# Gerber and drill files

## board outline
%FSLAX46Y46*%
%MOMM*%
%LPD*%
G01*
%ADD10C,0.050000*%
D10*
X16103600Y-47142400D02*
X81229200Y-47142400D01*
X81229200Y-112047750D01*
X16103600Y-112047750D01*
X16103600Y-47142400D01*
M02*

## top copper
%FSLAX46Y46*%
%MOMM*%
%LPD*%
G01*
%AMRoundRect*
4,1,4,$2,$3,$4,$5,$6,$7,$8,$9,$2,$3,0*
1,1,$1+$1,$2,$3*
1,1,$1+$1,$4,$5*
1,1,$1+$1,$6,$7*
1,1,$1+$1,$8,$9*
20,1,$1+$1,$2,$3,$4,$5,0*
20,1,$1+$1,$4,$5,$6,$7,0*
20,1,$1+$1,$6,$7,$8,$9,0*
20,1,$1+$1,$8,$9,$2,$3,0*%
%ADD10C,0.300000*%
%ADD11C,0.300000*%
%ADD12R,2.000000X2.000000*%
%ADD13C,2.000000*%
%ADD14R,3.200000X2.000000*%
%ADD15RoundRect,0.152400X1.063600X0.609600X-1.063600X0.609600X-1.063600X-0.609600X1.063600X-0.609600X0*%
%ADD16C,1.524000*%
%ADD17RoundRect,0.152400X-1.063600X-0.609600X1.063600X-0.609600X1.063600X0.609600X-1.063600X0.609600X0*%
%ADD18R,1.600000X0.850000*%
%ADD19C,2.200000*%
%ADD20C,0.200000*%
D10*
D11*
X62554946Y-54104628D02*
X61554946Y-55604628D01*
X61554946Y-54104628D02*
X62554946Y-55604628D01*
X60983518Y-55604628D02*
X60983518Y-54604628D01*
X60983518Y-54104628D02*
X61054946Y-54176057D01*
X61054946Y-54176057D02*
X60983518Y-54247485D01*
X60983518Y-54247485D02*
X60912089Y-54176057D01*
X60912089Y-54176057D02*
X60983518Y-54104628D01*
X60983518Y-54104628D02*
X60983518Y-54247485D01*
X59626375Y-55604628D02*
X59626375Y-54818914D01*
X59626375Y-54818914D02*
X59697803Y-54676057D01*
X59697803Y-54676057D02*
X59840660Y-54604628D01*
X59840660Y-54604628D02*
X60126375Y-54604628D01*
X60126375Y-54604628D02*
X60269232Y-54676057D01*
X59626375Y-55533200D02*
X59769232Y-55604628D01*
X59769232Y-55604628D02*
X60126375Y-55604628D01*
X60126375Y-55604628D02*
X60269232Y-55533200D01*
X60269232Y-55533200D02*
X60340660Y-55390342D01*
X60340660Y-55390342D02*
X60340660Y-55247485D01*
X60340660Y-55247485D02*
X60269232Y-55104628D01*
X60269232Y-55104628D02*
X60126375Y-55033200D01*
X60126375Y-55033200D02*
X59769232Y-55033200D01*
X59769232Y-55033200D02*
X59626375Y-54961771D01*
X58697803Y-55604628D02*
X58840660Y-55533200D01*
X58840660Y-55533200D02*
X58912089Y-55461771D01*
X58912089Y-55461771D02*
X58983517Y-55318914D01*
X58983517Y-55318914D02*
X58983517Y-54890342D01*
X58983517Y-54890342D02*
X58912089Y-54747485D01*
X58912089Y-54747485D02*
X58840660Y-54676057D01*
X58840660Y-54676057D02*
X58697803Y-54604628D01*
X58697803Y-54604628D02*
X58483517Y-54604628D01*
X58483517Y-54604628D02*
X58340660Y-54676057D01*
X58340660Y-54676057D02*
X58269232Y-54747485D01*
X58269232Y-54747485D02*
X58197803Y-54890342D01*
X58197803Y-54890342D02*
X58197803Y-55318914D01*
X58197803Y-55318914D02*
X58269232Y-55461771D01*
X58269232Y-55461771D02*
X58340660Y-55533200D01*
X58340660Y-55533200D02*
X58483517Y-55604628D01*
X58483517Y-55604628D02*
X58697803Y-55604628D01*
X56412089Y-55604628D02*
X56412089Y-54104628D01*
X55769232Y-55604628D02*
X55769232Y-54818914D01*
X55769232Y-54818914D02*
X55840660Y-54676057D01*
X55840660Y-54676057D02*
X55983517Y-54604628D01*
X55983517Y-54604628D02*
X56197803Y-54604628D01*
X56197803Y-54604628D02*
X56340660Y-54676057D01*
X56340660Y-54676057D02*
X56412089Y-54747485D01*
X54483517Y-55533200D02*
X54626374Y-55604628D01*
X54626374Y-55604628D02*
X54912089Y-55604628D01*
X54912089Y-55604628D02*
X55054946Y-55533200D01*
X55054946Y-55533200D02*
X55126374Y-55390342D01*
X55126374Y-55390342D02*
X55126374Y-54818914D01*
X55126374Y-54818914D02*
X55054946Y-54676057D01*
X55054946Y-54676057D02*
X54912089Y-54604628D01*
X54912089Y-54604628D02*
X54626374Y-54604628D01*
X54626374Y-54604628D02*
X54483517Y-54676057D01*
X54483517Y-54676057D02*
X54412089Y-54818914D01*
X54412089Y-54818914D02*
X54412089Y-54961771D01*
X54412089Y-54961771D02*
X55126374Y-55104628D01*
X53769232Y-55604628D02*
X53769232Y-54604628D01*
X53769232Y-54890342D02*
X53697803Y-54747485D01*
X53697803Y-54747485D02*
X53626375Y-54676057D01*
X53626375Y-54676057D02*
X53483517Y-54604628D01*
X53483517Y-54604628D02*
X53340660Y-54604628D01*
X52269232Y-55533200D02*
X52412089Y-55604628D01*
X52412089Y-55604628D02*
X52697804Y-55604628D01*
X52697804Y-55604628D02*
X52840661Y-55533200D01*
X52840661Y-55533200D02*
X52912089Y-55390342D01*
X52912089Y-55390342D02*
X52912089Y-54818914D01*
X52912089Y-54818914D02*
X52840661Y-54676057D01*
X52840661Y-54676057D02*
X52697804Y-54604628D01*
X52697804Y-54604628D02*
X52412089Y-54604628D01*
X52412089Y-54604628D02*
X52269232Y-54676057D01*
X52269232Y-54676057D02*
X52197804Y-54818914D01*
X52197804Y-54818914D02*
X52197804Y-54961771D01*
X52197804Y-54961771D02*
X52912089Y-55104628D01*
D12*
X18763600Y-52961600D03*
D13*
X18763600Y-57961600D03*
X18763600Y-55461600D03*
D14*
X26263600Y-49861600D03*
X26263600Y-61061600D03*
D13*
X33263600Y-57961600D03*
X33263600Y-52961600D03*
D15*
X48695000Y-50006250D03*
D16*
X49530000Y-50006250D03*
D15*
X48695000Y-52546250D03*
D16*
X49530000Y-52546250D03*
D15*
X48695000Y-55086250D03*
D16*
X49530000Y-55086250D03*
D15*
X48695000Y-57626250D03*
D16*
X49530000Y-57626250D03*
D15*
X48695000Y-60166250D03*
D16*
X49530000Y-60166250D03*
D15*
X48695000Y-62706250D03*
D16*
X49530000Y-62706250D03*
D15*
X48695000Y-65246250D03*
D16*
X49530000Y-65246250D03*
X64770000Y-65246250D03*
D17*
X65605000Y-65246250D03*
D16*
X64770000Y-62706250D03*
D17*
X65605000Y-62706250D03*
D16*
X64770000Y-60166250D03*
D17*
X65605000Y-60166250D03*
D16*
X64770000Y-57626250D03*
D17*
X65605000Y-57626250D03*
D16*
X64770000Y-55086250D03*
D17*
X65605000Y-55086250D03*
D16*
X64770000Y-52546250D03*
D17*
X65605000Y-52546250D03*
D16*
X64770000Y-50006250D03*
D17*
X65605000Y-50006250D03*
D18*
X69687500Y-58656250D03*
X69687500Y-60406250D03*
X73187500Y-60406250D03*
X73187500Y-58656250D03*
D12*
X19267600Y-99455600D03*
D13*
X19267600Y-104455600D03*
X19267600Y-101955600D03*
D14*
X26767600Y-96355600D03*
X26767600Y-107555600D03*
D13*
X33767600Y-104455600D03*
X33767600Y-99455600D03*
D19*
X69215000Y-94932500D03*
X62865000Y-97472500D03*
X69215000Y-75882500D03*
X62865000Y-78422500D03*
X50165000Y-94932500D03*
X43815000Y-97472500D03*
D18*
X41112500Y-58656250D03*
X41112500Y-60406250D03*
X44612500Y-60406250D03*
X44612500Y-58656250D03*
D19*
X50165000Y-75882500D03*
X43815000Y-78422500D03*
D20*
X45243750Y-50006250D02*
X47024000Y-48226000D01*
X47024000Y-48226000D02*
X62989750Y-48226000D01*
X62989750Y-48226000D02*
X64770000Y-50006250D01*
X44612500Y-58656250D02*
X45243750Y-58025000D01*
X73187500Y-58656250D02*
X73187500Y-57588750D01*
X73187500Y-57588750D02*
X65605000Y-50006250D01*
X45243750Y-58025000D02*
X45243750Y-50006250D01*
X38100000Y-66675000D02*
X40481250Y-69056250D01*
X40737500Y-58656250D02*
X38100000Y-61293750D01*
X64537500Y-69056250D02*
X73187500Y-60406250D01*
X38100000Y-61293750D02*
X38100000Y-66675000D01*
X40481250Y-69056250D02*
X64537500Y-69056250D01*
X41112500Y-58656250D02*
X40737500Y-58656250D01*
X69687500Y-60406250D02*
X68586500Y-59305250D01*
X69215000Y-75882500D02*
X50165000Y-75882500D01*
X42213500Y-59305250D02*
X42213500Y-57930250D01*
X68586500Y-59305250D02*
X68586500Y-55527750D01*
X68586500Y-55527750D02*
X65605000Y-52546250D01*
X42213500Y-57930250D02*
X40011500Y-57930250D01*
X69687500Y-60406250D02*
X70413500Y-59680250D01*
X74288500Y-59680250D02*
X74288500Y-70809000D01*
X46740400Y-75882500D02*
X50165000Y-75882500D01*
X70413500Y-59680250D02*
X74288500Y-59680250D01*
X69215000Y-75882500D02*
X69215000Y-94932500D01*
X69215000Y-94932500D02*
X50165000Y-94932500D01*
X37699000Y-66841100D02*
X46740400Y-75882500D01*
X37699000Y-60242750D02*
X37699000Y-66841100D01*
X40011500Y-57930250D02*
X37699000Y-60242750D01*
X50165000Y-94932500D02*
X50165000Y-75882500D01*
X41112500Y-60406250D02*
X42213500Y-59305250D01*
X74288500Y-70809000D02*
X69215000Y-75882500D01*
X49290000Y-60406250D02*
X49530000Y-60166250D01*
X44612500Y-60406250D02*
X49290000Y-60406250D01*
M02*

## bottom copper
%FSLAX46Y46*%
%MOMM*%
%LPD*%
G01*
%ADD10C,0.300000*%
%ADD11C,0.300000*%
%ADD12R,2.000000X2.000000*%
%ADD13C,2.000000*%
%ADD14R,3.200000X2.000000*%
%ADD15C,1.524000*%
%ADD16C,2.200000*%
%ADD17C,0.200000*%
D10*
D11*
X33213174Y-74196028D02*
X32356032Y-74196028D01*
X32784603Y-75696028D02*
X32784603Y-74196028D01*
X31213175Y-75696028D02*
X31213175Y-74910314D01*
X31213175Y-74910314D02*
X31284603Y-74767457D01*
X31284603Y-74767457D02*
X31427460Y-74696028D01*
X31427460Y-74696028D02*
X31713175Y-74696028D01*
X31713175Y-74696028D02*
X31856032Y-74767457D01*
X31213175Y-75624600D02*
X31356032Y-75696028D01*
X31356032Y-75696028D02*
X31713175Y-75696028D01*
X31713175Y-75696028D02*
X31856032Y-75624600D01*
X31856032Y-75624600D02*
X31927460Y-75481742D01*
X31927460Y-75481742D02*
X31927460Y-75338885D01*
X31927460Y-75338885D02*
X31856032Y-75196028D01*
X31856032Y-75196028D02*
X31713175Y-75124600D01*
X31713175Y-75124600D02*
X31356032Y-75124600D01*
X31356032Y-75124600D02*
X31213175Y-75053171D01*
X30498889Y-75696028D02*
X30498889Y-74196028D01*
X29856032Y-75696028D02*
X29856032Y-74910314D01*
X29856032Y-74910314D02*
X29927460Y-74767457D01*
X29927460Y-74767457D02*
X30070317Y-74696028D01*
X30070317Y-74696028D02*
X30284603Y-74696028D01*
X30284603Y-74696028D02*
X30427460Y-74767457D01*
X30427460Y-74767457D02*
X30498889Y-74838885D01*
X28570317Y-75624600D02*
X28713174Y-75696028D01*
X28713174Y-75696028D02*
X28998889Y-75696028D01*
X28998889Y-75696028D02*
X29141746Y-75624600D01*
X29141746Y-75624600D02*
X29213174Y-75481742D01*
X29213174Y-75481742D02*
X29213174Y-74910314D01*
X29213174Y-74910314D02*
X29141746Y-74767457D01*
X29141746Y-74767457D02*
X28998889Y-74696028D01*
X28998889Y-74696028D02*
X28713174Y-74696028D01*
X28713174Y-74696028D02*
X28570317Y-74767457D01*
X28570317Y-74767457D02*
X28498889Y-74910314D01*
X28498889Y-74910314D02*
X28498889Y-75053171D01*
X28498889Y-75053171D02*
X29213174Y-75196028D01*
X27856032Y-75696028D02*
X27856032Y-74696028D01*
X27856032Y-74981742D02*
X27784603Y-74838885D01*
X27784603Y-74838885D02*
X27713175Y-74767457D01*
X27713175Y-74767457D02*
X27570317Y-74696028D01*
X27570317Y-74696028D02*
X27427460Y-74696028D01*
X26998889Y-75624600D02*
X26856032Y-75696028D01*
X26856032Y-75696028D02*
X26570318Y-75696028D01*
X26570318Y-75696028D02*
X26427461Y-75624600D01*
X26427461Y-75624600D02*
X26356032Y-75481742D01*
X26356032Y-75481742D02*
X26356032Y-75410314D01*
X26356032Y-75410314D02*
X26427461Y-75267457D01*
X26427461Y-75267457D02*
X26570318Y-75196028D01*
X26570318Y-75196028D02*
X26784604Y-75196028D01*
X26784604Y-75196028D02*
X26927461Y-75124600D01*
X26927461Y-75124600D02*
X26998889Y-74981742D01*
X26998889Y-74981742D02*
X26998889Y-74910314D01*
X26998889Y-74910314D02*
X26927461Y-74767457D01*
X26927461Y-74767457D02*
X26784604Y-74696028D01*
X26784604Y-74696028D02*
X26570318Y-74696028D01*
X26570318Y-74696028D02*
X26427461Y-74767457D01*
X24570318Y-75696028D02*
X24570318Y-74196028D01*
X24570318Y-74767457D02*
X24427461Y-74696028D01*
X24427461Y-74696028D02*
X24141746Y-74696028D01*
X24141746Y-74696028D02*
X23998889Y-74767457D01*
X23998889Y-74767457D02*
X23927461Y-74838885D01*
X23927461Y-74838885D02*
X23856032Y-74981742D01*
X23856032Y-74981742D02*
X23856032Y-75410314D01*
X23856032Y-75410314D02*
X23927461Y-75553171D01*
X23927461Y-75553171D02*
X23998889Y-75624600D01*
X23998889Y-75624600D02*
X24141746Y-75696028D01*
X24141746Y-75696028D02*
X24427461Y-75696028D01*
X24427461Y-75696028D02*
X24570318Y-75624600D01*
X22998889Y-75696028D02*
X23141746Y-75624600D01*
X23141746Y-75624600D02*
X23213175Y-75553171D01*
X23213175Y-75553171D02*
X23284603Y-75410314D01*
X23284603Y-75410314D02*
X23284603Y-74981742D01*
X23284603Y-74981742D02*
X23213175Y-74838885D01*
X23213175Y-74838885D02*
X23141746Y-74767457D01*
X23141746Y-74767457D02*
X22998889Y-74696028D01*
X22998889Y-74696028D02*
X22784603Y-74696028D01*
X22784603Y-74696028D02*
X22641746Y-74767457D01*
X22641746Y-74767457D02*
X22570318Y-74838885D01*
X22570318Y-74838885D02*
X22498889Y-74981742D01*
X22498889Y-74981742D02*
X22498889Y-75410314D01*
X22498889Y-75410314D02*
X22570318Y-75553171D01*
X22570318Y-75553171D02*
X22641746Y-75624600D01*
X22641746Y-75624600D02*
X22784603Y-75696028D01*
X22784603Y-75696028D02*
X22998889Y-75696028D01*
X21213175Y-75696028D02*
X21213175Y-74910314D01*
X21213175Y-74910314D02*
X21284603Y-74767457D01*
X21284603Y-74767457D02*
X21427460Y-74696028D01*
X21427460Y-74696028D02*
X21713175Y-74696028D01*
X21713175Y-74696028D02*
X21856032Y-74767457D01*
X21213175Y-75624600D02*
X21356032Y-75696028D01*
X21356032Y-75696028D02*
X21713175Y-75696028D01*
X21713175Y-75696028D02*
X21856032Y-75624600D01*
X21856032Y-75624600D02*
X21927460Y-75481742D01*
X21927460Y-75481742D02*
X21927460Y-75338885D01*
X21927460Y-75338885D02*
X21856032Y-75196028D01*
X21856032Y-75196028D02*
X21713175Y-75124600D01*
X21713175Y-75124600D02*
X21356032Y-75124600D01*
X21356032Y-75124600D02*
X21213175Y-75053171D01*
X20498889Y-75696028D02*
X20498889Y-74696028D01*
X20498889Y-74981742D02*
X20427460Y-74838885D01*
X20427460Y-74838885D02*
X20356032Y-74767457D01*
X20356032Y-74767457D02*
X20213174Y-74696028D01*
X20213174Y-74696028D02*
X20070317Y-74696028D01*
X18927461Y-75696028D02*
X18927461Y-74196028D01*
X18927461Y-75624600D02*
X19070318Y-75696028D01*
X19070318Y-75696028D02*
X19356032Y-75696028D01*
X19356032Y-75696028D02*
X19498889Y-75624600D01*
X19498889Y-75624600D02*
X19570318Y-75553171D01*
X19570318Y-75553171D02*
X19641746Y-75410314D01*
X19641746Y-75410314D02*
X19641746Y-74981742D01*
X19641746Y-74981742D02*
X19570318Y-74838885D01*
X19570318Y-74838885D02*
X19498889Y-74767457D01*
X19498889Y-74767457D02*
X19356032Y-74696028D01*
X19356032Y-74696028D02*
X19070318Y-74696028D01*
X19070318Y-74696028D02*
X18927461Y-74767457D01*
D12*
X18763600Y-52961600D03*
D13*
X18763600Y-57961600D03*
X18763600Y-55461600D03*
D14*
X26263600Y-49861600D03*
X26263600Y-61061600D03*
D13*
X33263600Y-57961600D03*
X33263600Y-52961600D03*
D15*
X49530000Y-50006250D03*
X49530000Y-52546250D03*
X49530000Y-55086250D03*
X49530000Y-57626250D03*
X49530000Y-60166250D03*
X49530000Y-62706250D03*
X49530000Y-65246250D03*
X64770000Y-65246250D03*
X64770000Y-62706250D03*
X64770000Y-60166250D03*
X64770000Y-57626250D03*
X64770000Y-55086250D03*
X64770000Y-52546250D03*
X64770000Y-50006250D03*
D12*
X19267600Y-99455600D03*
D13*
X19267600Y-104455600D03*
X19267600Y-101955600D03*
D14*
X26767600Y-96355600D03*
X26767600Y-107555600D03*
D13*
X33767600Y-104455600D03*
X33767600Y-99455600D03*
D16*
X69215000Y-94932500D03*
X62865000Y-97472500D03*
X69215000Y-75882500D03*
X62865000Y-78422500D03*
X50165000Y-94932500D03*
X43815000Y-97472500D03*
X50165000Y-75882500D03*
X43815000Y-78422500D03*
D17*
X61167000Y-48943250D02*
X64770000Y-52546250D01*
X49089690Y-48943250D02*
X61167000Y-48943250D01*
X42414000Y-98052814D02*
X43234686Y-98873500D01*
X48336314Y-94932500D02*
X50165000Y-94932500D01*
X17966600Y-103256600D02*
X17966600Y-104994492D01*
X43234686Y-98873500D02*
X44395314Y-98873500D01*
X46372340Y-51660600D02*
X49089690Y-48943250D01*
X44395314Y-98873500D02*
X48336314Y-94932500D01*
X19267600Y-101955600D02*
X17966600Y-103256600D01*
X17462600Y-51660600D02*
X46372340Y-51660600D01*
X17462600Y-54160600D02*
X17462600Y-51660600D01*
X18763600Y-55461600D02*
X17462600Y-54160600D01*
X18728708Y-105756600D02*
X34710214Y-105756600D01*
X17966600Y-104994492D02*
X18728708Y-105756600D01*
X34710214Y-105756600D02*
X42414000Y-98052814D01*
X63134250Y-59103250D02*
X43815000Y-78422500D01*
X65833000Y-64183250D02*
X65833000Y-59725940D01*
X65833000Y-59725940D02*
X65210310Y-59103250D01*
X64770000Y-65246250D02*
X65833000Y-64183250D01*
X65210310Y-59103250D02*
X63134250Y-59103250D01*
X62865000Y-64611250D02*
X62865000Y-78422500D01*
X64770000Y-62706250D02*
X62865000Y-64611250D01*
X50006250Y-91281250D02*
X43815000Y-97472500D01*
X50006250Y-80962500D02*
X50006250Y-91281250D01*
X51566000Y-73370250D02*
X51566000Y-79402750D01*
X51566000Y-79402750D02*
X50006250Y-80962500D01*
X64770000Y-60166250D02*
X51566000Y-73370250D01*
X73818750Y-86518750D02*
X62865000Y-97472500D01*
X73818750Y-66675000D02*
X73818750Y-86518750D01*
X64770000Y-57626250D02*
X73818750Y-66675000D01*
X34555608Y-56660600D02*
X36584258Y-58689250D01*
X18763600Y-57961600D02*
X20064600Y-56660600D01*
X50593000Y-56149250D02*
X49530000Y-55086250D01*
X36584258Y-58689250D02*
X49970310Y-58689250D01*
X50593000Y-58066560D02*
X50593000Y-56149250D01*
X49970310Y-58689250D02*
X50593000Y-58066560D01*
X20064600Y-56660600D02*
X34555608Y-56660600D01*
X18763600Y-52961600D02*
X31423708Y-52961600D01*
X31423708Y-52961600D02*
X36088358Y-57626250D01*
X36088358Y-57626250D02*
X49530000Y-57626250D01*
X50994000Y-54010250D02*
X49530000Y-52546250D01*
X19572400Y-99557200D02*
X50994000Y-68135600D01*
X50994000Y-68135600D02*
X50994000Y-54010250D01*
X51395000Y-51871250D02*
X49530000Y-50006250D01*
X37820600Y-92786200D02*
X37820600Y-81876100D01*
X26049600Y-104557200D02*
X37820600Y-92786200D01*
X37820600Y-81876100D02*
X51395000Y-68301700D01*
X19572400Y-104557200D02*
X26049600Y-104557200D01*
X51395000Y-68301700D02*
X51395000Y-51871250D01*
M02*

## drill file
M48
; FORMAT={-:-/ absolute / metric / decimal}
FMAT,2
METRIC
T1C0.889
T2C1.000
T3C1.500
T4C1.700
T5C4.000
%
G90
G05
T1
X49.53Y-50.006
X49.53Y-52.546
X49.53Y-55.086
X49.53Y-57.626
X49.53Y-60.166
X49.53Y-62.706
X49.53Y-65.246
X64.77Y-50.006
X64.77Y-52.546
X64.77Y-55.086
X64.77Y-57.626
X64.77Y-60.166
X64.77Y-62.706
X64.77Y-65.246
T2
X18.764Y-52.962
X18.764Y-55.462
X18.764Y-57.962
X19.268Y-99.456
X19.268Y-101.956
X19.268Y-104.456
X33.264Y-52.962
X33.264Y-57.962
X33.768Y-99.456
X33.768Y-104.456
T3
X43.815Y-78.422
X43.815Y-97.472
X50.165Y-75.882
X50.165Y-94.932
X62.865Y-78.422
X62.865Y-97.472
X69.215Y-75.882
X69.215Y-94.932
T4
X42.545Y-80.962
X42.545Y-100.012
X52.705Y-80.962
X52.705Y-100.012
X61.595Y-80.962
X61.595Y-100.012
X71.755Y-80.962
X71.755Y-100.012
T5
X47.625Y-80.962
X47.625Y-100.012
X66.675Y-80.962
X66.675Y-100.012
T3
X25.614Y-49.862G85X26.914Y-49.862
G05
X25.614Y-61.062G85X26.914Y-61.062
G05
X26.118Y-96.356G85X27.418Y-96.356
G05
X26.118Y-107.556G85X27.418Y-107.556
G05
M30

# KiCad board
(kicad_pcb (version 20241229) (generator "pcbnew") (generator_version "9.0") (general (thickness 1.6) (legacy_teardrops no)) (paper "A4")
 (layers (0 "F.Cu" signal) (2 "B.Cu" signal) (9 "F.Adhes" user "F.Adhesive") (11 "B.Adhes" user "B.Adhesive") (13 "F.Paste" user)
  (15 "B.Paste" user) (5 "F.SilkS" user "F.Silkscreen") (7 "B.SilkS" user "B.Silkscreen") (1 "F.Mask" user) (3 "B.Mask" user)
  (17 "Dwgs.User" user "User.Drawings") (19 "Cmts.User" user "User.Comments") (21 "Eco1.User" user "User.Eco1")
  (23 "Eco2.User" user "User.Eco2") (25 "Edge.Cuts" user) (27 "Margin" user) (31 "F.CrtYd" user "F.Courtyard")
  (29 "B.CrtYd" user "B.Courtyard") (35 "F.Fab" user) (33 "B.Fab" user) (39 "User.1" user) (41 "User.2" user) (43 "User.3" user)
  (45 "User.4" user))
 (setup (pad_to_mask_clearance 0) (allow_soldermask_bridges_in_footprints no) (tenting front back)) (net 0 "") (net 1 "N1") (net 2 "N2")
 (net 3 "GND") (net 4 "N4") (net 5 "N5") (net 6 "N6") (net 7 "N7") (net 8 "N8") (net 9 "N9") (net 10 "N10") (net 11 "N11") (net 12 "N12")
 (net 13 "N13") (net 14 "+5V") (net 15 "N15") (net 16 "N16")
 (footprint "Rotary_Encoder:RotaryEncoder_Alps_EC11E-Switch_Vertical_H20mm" (layer "F.Cu") (at 18.7636 52.9616)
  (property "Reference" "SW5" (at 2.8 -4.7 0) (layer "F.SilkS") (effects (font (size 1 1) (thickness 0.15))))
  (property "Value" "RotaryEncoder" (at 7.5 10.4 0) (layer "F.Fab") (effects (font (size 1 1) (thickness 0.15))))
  (pad "A" thru_hole rect (at 0 0) (size 2 2) (drill 1) (layers "*.Cu" "*.Mask") (remove_unused_layers no) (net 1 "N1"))
  (pad "B" thru_hole circle (at 0 5) (size 2 2) (drill 1) (layers "*.Cu" "*.Mask") (remove_unused_layers no) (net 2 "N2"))
  (pad "C" thru_hole circle (at 0 2.5) (size 2 2) (drill 1) (layers "*.Cu" "*.Mask") (remove_unused_layers no) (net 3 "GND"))
  (pad "MP" thru_hole rect (at 7.5 -3.1) (size 3.2 2) (drill oval 2.8 1.5) (layers "*.Cu" "*.Mask") (remove_unused_layers no))
  (pad "MP" thru_hole rect (at 7.5 8.1) (size 3.2 2) (drill oval 2.8 1.5) (layers "*.Cu" "*.Mask") (remove_unused_layers no))
  (pad "S1" thru_hole circle (at 14.5 5) (size 2 2) (drill 1) (layers "*.Cu" "*.Mask") (remove_unused_layers no))
  (pad "S2" thru_hole circle (at 14.5 0) (size 2 2) (drill 1) (layers "*.Cu" "*.Mask") (remove_unused_layers no)))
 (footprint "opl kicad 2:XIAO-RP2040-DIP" (layer "F.Cu") (at 57.15 57.62625)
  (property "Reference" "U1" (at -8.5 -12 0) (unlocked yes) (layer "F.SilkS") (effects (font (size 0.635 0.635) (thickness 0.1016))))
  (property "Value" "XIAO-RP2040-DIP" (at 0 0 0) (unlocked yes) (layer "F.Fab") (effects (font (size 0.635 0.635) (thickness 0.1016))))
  (pad "1" smd roundrect (at -8.455 -7.62 180) (size 2.432 1.524) (layers "F.Cu" "F.Mask") (roundrect_rratio 0.1) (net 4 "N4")
   (thermal_bridge_angle 45))
  (pad "1" thru_hole circle (at -7.62 -7.62 180) (size 1.524 1.524) (drill 0.889) (layers "*.Cu" "*.Mask") (remove_unused_layers no)
   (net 4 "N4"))
  (pad "2" smd roundrect (at -8.455 -5.08 180) (size 2.432 1.524) (layers "F.Cu" "F.Mask") (roundrect_rratio 0.1) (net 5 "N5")
   (thermal_bridge_angle 45))
  (pad "2" thru_hole circle (at -7.62 -5.08 180) (size 1.524 1.524) (drill 0.889) (layers "*.Cu" "*.Mask") (remove_unused_layers no)
   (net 5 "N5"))
  (pad "3" smd roundrect (at -8.455 -2.54 180) (size 2.432 1.524) (layers "F.Cu" "F.Mask") (roundrect_rratio 0.1) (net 2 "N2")
   (thermal_bridge_angle 45))
  (pad "3" thru_hole circle (at -7.62 -2.54 180) (size 1.524 1.524) (drill 0.889) (layers "*.Cu" "*.Mask") (remove_unused_layers no)
   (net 2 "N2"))
  (pad "4" smd roundrect (at -8.455 0 180) (size 2.432 1.524) (layers "F.Cu" "F.Mask") (roundrect_rratio 0.1) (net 1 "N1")
   (thermal_bridge_angle 45))
  (pad "4" thru_hole circle (at -7.62 0 180) (size 1.524 1.524) (drill 0.889) (layers "*.Cu" "*.Mask") (remove_unused_layers no)
   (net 1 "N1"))
  (pad "5" smd roundrect (at -8.455 2.54 180) (size 2.432 1.524) (layers "F.Cu" "F.Mask") (roundrect_rratio 0.1) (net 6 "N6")
   (thermal_bridge_angle 45))
  (pad "5" thru_hole circle (at -7.62 2.54 180) (size 1.524 1.524) (drill 0.889) (layers "*.Cu" "*.Mask") (remove_unused_layers no)
   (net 6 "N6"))
  (pad "6" smd roundrect (at -8.455 5.08 180) (size 2.432 1.524) (layers "F.Cu" "F.Mask") (roundrect_rratio 0.1) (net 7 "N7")
   (thermal_bridge_angle 45))
  (pad "6" thru_hole circle (at -7.62 5.08 180) (size 1.524 1.524) (drill 0.889) (layers "*.Cu" "*.Mask") (remove_unused_layers no)
   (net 7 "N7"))
  (pad "7" smd roundrect (at -8.455 7.62 180) (size 2.432 1.524) (layers "F.Cu" "F.Mask") (roundrect_rratio 0.1) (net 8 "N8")
   (thermal_bridge_angle 45))
  (pad "7" thru_hole circle (at -7.62 7.62 180) (size 1.524 1.524) (drill 0.889) (layers "*.Cu" "*.Mask") (remove_unused_layers no)
   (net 8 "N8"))
  (pad "8" thru_hole circle (at 7.62 7.62) (size 1.524 1.524) (drill 0.889) (layers "*.Cu" "*.Mask") (remove_unused_layers no) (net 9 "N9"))
  (pad "8" smd roundrect (at 8.455 7.62) (size 2.432 1.524) (layers "F.Cu" "F.Mask") (roundrect_rratio 0.1) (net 9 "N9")
   (thermal_bridge_angle 45))
  (pad "9" thru_hole circle (at 7.62 5.08) (size 1.524 1.524) (drill 0.889) (layers "*.Cu" "*.Mask") (remove_unused_layers no)
   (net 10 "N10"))
  (pad "9" smd roundrect (at 8.455 5.08) (size 2.432 1.524) (layers "F.Cu" "F.Mask") (roundrect_rratio 0.1) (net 10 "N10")
   (thermal_bridge_angle 45))
  (pad "10" thru_hole circle (at 7.62 2.54) (size 1.524 1.524) (drill 0.889) (layers "*.Cu" "*.Mask") (remove_unused_layers no)
   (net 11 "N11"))
  (pad "10" smd roundrect (at 8.455 2.54) (size 2.432 1.524) (layers "F.Cu" "F.Mask") (roundrect_rratio 0.1) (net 11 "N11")
   (thermal_bridge_angle 45))
  (pad "11" thru_hole circle (at 7.62 0) (size 1.524 1.524) (drill 0.889) (layers "*.Cu" "*.Mask") (remove_unused_layers no) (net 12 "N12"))
  (pad "11" smd roundrect (at 8.455 0) (size 2.432 1.524) (layers "F.Cu" "F.Mask") (roundrect_rratio 0.1) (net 12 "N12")
   (thermal_bridge_angle 45))
  (pad "12" thru_hole circle (at 7.62 -2.54) (size 1.524 1.524) (drill 0.889) (layers "*.Cu" "*.Mask") (remove_unused_layers no)
   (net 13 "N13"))
  (pad "12" smd roundrect (at 8.455 -2.54) (size 2.432 1.524) (layers "F.Cu" "F.Mask") (roundrect_rratio 0.1) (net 13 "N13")
   (thermal_bridge_angle 45))
  (pad "13" thru_hole circle (at 7.62 -5.08) (size 1.524 1.524) (drill 0.889) (layers "*.Cu" "*.Mask") (remove_unused_layers no)
   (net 3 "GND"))
  (pad "13" smd roundrect (at 8.455 -5.08) (size 2.432 1.524) (layers "F.Cu" "F.Mask") (roundrect_rratio 0.1) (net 3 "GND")
   (thermal_bridge_angle 45))
  (pad "14" thru_hole circle (at 7.62 -7.62) (size 1.524 1.524) (drill 0.889) (layers "*.Cu" "*.Mask") (remove_unused_layers no)
   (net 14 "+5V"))
  (pad "14" smd roundrect (at 8.455 -7.62) (size 2.432 1.524) (layers "F.Cu" "F.Mask") (roundrect_rratio 0.1) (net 14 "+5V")
   (thermal_bridge_angle 45)))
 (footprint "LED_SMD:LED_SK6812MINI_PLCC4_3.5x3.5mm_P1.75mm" (layer "F.Cu") (at 71.4375 59.53125)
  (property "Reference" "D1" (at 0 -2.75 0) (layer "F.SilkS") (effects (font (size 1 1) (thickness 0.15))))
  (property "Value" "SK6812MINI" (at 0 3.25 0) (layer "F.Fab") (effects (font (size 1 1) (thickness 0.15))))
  (pad "1" smd rect (at -1.75 -0.875) (size 1.6 0.85) (layers "F.Cu" "F.Mask" "F.Paste") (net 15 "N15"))
  (pad "2" smd rect (at -1.75 0.875) (size 1.6 0.85) (layers "F.Cu" "F.Mask" "F.Paste") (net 3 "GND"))
  (pad "3" smd rect (at 1.75 0.875) (size 1.6 0.85) (layers "F.Cu" "F.Mask" "F.Paste") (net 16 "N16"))
  (pad "4" smd rect (at 1.75 -0.875) (size 1.6 0.85) (layers "F.Cu" "F.Mask" "F.Paste") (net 14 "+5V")))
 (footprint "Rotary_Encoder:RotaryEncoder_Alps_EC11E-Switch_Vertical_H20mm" (layer "F.Cu") (at 19.2676 99.4556)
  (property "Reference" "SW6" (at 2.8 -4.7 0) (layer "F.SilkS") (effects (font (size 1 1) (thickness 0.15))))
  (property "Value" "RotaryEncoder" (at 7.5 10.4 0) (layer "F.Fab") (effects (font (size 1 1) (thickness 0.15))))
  (pad "A" thru_hole rect (at 0 0) (size 2 2) (drill 1) (layers "*.Cu" "*.Mask") (remove_unused_layers no) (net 5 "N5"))
  (pad "B" thru_hole circle (at 0 5) (size 2 2) (drill 1) (layers "*.Cu" "*.Mask") (remove_unused_layers no) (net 4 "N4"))
  (pad "C" thru_hole circle (at 0 2.5) (size 2 2) (drill 1) (layers "*.Cu" "*.Mask") (remove_unused_layers no) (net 3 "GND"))
  (pad "MP" thru_hole rect (at 7.5 -3.1) (size 3.2 2) (drill oval 2.8 1.5) (layers "*.Cu" "*.Mask") (remove_unused_layers no))
  (pad "MP" thru_hole rect (at 7.5 8.1) (size 3.2 2) (drill oval 2.8 1.5) (layers "*.Cu" "*.Mask") (remove_unused_layers no))
  (pad "S1" thru_hole circle (at 14.5 5) (size 2 2) (drill 1) (layers "*.Cu" "*.Mask") (remove_unused_layers no))
  (pad "S2" thru_hole circle (at 14.5 0) (size 2 2) (drill 1) (layers "*.Cu" "*.Mask") (remove_unused_layers no)))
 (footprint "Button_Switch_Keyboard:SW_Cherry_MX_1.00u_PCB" (layer "F.Cu") (at 69.215 94.9325)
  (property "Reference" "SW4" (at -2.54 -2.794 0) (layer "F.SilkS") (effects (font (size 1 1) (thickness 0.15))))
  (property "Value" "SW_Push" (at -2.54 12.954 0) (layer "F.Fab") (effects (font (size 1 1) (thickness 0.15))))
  (pad "" np_thru_hole circle (at -7.62 5.08) (size 1.7 1.7) (drill 1.7) (layers "*.Cu" "*.Mask"))
  (pad "" np_thru_hole circle (at -2.54 5.08) (size 4 4) (drill 4) (layers "*.Cu" "*.Mask"))
  (pad "" np_thru_hole circle (at 2.54 5.08) (size 1.7 1.7) (drill 1.7) (layers "*.Cu" "*.Mask"))
  (pad "1" thru_hole circle (at 0 0) (size 2.2 2.2) (drill 1.5) (layers "*.Cu" "*.Mask") (remove_unused_layers no) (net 3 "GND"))
  (pad "2" thru_hole circle (at -6.35 2.54) (size 2.2 2.2) (drill 1.5) (layers "*.Cu" "*.Mask") (remove_unused_layers no) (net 12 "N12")))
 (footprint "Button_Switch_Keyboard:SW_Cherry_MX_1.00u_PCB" (layer "F.Cu") (at 69.215 75.8825)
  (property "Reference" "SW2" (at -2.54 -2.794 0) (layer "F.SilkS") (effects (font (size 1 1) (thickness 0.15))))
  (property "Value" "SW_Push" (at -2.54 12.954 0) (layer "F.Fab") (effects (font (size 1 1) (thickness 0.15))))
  (pad "" np_thru_hole circle (at -7.62 5.08) (size 1.7 1.7) (drill 1.7) (layers "*.Cu" "*.Mask"))
  (pad "" np_thru_hole circle (at -2.54 5.08) (size 4 4) (drill 4) (layers "*.Cu" "*.Mask"))
  (pad "" np_thru_hole circle (at 2.54 5.08) (size 1.7 1.7) (drill 1.7) (layers "*.Cu" "*.Mask"))
  (pad "1" thru_hole circle (at 0 0) (size 2.2 2.2) (drill 1.5) (layers "*.Cu" "*.Mask") (remove_unused_layers no) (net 3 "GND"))
  (pad "2" thru_hole circle (at -6.35 2.54) (size 2.2 2.2) (drill 1.5) (layers "*.Cu" "*.Mask") (remove_unused_layers no) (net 10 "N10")))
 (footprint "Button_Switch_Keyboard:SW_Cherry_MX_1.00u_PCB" (layer "F.Cu") (at 50.165 94.9325)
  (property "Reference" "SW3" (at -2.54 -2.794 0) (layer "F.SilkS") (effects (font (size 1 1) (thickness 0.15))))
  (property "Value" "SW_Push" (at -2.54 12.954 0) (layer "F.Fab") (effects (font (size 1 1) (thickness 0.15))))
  (pad "" np_thru_hole circle (at -7.62 5.08) (size 1.7 1.7) (drill 1.7) (layers "*.Cu" "*.Mask"))
  (pad "" np_thru_hole circle (at -2.54 5.08) (size 4 4) (drill 4) (layers "*.Cu" "*.Mask"))
  (pad "" np_thru_hole circle (at 2.54 5.08) (size 1.7 1.7) (drill 1.7) (layers "*.Cu" "*.Mask"))
  (pad "1" thru_hole circle (at 0 0) (size 2.2 2.2) (drill 1.5) (layers "*.Cu" "*.Mask") (remove_unused_layers no) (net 3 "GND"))
  (pad "2" thru_hole circle (at -6.35 2.54) (size 2.2 2.2) (drill 1.5) (layers "*.Cu" "*.Mask") (remove_unused_layers no) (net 11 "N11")))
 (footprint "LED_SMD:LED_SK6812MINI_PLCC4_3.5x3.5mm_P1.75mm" (layer "F.Cu") (at 42.8625 59.53125)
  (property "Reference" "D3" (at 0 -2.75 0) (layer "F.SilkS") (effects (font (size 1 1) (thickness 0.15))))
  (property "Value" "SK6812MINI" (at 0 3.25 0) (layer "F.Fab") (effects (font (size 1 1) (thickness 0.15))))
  (pad "1" smd rect (at -1.75 -0.875) (size 1.6 0.85) (layers "F.Cu" "F.Mask" "F.Paste") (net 16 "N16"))
  (pad "2" smd rect (at -1.75 0.875) (size 1.6 0.85) (layers "F.Cu" "F.Mask" "F.Paste") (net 3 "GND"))
  (pad "3" smd rect (at 1.75 0.875) (size 1.6 0.85) (layers "F.Cu" "F.Mask" "F.Paste") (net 6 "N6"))
  (pad "4" smd rect (at 1.75 -0.875) (size 1.6 0.85) (layers "F.Cu" "F.Mask" "F.Paste") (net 14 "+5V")))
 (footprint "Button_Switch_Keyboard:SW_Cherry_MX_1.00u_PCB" (layer "F.Cu") (at 50.165 75.8825)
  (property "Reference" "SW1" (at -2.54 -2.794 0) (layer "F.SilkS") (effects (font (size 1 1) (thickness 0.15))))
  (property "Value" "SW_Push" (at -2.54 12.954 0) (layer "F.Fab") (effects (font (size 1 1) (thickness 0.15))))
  (pad "" np_thru_hole circle (at -7.62 5.08) (size 1.7 1.7) (drill 1.7) (layers "*.Cu" "*.Mask"))
  (pad "" np_thru_hole circle (at -2.54 5.08) (size 4 4) (drill 4) (layers "*.Cu" "*.Mask"))
  (pad "" np_thru_hole circle (at 2.54 5.08) (size 1.7 1.7) (drill 1.7) (layers "*.Cu" "*.Mask"))
  (pad "1" thru_hole circle (at 0 0) (size 2.2 2.2) (drill 1.5) (layers "*.Cu" "*.Mask") (remove_unused_layers no) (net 3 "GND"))
  (pad "2" thru_hole circle (at -6.35 2.54) (size 2.2 2.2) (drill 1.5) (layers "*.Cu" "*.Mask") (remove_unused_layers no) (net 9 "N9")))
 (gr_rect (start 16.1036 47.1424) (end 81.2292 112.04775) (stroke (width 0.05) (type default)) (fill no) (layer "Edge.Cuts"))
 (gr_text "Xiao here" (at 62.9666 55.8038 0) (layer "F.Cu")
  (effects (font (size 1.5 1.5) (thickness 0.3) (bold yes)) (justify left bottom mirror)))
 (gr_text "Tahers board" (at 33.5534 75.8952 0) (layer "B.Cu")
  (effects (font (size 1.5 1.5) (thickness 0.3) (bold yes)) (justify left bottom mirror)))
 (segment (start 45.24375 50.00625) (end 47.024 48.226) (width 0.2) (layer "F.Cu") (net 14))
 (segment (start 47.024 48.226) (end 62.98975 48.226) (width 0.2) (layer "F.Cu") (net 14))
 (segment (start 62.98975 48.226) (end 64.77 50.00625) (width 0.2) (layer "F.Cu") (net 14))
 (segment (start 44.6125 58.65625) (end 45.24375 58.025) (width 0.2) (layer "F.Cu") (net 14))
 (segment (start 73.1875 58.65625) (end 73.1875 57.58875) (width 0.2) (layer "F.Cu") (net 14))
 (segment (start 73.1875 57.58875) (end 65.605 50.00625) (width 0.2) (layer "F.Cu") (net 14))
 (segment (start 45.24375 58.025) (end 45.24375 50.00625) (width 0.2) (layer "F.Cu") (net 14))
 (segment (start 38.1 66.675) (end 40.48125 69.05625) (width 0.2) (layer "F.Cu") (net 16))
 (segment (start 40.7375 58.65625) (end 38.1 61.29375) (width 0.2) (layer "F.Cu") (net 16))
 (segment (start 64.5375 69.05625) (end 73.1875 60.40625) (width 0.2) (layer "F.Cu") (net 16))
 (segment (start 38.1 61.29375) (end 38.1 66.675) (width 0.2) (layer "F.Cu") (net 16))
 (segment (start 40.48125 69.05625) (end 64.5375 69.05625) (width 0.2) (layer "F.Cu") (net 16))
 (segment (start 41.1125 58.65625) (end 40.7375 58.65625) (width 0.2) (layer "F.Cu") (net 16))
 (segment (start 69.6875 60.40625) (end 68.5865 59.30525) (width 0.2) (layer "F.Cu") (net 3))
 (segment (start 69.215 75.8825) (end 50.165 75.8825) (width 0.2) (layer "F.Cu") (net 3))
 (segment (start 42.2135 59.30525) (end 42.2135 57.93025) (width 0.2) (layer "F.Cu") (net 3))
 (segment (start 68.5865 59.30525) (end 68.5865 55.52775) (width 0.2) (layer "F.Cu") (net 3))
 (segment (start 68.5865 55.52775) (end 65.605 52.54625) (width 0.2) (layer "F.Cu") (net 3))
 (segment (start 42.2135 57.93025) (end 40.0115 57.93025) (width 0.2) (layer "F.Cu") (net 3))
 (segment (start 69.6875 60.40625) (end 70.4135 59.68025) (width 0.2) (layer "F.Cu") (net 3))
 (segment (start 74.2885 59.68025) (end 74.2885 70.809) (width 0.2) (layer "F.Cu") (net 3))
 (segment (start 46.7404 75.8825) (end 50.165 75.8825) (width 0.2) (layer "F.Cu") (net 3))
 (segment (start 70.4135 59.68025) (end 74.2885 59.68025) (width 0.2) (layer "F.Cu") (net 3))
 (segment (start 69.215 75.8825) (end 69.215 94.9325) (width 0.2) (layer "F.Cu") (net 3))
 (segment (start 69.215 94.9325) (end 50.165 94.9325) (width 0.2) (layer "F.Cu") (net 3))
 (segment (start 37.699 66.8411) (end 46.7404 75.8825) (width 0.2) (layer "F.Cu") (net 3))
 (segment (start 37.699 60.24275) (end 37.699 66.8411) (width 0.2) (layer "F.Cu") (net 3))
 (segment (start 40.0115 57.93025) (end 37.699 60.24275) (width 0.2) (layer "F.Cu") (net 3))
 (segment (start 50.165 94.9325) (end 50.165 75.8825) (width 0.2) (layer "F.Cu") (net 3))
 (segment (start 41.1125 60.40625) (end 42.2135 59.30525) (width 0.2) (layer "F.Cu") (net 3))
 (segment (start 74.2885 70.809) (end 69.215 75.8825) (width 0.2) (layer "F.Cu") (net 3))
 (segment (start 61.167 48.94325) (end 64.77 52.54625) (width 0.2) (layer "B.Cu") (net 3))
 (segment (start 49.08969 48.94325) (end 61.167 48.94325) (width 0.2) (layer "B.Cu") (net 3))
 (segment (start 42.414 98.052814) (end 43.234686 98.8735) (width 0.2) (layer "B.Cu") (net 3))
 (segment (start 48.336314 94.9325) (end 50.165 94.9325) (width 0.2) (layer "B.Cu") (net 3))
 (segment (start 17.9666 103.2566) (end 17.9666 104.994492) (width 0.2) (layer "B.Cu") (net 3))
 (segment (start 43.234686 98.8735) (end 44.395314 98.8735) (width 0.2) (layer "B.Cu") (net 3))
 (segment (start 46.37234 51.6606) (end 49.08969 48.94325) (width 0.2) (layer "B.Cu") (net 3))
 (segment (start 44.395314 98.8735) (end 48.336314 94.9325) (width 0.2) (layer "B.Cu") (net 3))
 (segment (start 19.2676 101.9556) (end 17.9666 103.2566) (width 0.2) (layer "B.Cu") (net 3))
 (segment (start 17.4626 51.6606) (end 46.37234 51.6606) (width 0.2) (layer "B.Cu") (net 3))
 (segment (start 17.4626 54.1606) (end 17.4626 51.6606) (width 0.2) (layer "B.Cu") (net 3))
 (segment (start 18.7636 55.4616) (end 17.4626 54.1606) (width 0.2) (layer "B.Cu") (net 3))
 (segment (start 18.728708 105.7566) (end 34.710214 105.7566) (width 0.2) (layer "B.Cu") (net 3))
 (segment (start 17.9666 104.994492) (end 18.728708 105.7566) (width 0.2) (layer "B.Cu") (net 3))
 (segment (start 34.710214 105.7566) (end 42.414 98.052814) (width 0.2) (layer "B.Cu") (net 3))
 (segment (start 49.29 60.40625) (end 49.53 60.16625) (width 0.2) (layer "F.Cu") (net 6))
 (segment (start 44.6125 60.40625) (end 49.29 60.40625) (width 0.2) (layer "F.Cu") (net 6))
 (segment (start 63.13425 59.10325) (end 43.815 78.4225) (width 0.2) (layer "B.Cu") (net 9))
 (segment (start 65.833 64.18325) (end 65.833 59.72594) (width 0.2) (layer "B.Cu") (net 9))
 (segment (start 65.833 59.72594) (end 65.21031 59.10325) (width 0.2) (layer "B.Cu") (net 9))
 (segment (start 64.77 65.24625) (end 65.833 64.18325) (width 0.2) (layer "B.Cu") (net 9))
 (segment (start 65.21031 59.10325) (end 63.13425 59.10325) (width 0.2) (layer "B.Cu") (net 9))
 (segment (start 62.865 64.61125) (end 62.865 78.4225) (width 0.2) (layer "B.Cu") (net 10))
 (segment (start 64.77 62.70625) (end 62.865 64.61125) (width 0.2) (layer "B.Cu") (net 10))
 (segment (start 50.00625 91.28125) (end 43.815 97.4725) (width 0.2) (layer "B.Cu") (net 11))
 (segment (start 50.00625 80.9625) (end 50.00625 91.28125) (width 0.2) (layer "B.Cu") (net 11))
 (segment (start 51.566 73.37025) (end 51.566 79.40275) (width 0.2) (layer "B.Cu") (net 11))
 (segment (start 51.566 79.40275) (end 50.00625 80.9625) (width 0.2) (layer "B.Cu") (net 11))
 (segment (start 64.77 60.16625) (end 51.566 73.37025) (width 0.2) (layer "B.Cu") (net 11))
 (segment (start 73.81875 86.51875) (end 62.865 97.4725) (width 0.2) (layer "B.Cu") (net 12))
 (segment (start 73.81875 66.675) (end 73.81875 86.51875) (width 0.2) (layer "B.Cu") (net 12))
 (segment (start 64.77 57.62625) (end 73.81875 66.675) (width 0.2) (layer "B.Cu") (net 12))
 (segment (start 34.555608 56.6606) (end 36.584258 58.68925) (width 0.2) (layer "B.Cu") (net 2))
 (segment (start 18.7636 57.9616) (end 20.0646 56.6606) (width 0.2) (layer "B.Cu") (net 2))
 (segment (start 50.593 56.14925) (end 49.53 55.08625) (width 0.2) (layer "B.Cu") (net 2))
 (segment (start 36.584258 58.68925) (end 49.97031 58.68925) (width 0.2) (layer "B.Cu") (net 2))
 (segment (start 50.593 58.06656) (end 50.593 56.14925) (width 0.2) (layer "B.Cu") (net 2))
 (segment (start 49.97031 58.68925) (end 50.593 58.06656) (width 0.2) (layer "B.Cu") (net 2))
 (segment (start 20.0646 56.6606) (end 34.555608 56.6606) (width 0.2) (layer "B.Cu") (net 2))
 (segment (start 18.7636 52.9616) (end 31.423708 52.9616) (width 0.2) (layer "B.Cu") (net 1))
 (segment (start 31.423708 52.9616) (end 36.088358 57.62625) (width 0.2) (layer "B.Cu") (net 1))
 (segment (start 36.088358 57.62625) (end 49.53 57.62625) (width 0.2) (layer "B.Cu") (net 1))
 (segment (start 50.994 54.01025) (end 49.53 52.54625) (width 0.2) (layer "B.Cu") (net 5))
 (segment (start 19.5724 99.5572) (end 50.994 68.1356) (width 0.2) (layer "B.Cu") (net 5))
 (segment (start 50.994 68.1356) (end 50.994 54.01025) (width 0.2) (layer "B.Cu") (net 5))
 (segment (start 51.395 51.87125) (end 49.53 50.00625) (width 0.2) (layer "B.Cu") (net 4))
 (segment (start 37.8206 92.7862) (end 37.8206 81.8761) (width 0.2) (layer "B.Cu") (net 4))
 (segment (start 26.0496 104.5572) (end 37.8206 92.7862) (width 0.2) (layer "B.Cu") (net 4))
 (segment (start 37.8206 81.8761) (end 51.395 68.3017) (width 0.2) (layer "B.Cu") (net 4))
 (segment (start 19.5724 104.5572) (end 26.0496 104.5572) (width 0.2) (layer "B.Cu") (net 4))
 (segment (start 51.395 68.3017) (end 51.395 51.87125) (width 0.2) (layer "B.Cu") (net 4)))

